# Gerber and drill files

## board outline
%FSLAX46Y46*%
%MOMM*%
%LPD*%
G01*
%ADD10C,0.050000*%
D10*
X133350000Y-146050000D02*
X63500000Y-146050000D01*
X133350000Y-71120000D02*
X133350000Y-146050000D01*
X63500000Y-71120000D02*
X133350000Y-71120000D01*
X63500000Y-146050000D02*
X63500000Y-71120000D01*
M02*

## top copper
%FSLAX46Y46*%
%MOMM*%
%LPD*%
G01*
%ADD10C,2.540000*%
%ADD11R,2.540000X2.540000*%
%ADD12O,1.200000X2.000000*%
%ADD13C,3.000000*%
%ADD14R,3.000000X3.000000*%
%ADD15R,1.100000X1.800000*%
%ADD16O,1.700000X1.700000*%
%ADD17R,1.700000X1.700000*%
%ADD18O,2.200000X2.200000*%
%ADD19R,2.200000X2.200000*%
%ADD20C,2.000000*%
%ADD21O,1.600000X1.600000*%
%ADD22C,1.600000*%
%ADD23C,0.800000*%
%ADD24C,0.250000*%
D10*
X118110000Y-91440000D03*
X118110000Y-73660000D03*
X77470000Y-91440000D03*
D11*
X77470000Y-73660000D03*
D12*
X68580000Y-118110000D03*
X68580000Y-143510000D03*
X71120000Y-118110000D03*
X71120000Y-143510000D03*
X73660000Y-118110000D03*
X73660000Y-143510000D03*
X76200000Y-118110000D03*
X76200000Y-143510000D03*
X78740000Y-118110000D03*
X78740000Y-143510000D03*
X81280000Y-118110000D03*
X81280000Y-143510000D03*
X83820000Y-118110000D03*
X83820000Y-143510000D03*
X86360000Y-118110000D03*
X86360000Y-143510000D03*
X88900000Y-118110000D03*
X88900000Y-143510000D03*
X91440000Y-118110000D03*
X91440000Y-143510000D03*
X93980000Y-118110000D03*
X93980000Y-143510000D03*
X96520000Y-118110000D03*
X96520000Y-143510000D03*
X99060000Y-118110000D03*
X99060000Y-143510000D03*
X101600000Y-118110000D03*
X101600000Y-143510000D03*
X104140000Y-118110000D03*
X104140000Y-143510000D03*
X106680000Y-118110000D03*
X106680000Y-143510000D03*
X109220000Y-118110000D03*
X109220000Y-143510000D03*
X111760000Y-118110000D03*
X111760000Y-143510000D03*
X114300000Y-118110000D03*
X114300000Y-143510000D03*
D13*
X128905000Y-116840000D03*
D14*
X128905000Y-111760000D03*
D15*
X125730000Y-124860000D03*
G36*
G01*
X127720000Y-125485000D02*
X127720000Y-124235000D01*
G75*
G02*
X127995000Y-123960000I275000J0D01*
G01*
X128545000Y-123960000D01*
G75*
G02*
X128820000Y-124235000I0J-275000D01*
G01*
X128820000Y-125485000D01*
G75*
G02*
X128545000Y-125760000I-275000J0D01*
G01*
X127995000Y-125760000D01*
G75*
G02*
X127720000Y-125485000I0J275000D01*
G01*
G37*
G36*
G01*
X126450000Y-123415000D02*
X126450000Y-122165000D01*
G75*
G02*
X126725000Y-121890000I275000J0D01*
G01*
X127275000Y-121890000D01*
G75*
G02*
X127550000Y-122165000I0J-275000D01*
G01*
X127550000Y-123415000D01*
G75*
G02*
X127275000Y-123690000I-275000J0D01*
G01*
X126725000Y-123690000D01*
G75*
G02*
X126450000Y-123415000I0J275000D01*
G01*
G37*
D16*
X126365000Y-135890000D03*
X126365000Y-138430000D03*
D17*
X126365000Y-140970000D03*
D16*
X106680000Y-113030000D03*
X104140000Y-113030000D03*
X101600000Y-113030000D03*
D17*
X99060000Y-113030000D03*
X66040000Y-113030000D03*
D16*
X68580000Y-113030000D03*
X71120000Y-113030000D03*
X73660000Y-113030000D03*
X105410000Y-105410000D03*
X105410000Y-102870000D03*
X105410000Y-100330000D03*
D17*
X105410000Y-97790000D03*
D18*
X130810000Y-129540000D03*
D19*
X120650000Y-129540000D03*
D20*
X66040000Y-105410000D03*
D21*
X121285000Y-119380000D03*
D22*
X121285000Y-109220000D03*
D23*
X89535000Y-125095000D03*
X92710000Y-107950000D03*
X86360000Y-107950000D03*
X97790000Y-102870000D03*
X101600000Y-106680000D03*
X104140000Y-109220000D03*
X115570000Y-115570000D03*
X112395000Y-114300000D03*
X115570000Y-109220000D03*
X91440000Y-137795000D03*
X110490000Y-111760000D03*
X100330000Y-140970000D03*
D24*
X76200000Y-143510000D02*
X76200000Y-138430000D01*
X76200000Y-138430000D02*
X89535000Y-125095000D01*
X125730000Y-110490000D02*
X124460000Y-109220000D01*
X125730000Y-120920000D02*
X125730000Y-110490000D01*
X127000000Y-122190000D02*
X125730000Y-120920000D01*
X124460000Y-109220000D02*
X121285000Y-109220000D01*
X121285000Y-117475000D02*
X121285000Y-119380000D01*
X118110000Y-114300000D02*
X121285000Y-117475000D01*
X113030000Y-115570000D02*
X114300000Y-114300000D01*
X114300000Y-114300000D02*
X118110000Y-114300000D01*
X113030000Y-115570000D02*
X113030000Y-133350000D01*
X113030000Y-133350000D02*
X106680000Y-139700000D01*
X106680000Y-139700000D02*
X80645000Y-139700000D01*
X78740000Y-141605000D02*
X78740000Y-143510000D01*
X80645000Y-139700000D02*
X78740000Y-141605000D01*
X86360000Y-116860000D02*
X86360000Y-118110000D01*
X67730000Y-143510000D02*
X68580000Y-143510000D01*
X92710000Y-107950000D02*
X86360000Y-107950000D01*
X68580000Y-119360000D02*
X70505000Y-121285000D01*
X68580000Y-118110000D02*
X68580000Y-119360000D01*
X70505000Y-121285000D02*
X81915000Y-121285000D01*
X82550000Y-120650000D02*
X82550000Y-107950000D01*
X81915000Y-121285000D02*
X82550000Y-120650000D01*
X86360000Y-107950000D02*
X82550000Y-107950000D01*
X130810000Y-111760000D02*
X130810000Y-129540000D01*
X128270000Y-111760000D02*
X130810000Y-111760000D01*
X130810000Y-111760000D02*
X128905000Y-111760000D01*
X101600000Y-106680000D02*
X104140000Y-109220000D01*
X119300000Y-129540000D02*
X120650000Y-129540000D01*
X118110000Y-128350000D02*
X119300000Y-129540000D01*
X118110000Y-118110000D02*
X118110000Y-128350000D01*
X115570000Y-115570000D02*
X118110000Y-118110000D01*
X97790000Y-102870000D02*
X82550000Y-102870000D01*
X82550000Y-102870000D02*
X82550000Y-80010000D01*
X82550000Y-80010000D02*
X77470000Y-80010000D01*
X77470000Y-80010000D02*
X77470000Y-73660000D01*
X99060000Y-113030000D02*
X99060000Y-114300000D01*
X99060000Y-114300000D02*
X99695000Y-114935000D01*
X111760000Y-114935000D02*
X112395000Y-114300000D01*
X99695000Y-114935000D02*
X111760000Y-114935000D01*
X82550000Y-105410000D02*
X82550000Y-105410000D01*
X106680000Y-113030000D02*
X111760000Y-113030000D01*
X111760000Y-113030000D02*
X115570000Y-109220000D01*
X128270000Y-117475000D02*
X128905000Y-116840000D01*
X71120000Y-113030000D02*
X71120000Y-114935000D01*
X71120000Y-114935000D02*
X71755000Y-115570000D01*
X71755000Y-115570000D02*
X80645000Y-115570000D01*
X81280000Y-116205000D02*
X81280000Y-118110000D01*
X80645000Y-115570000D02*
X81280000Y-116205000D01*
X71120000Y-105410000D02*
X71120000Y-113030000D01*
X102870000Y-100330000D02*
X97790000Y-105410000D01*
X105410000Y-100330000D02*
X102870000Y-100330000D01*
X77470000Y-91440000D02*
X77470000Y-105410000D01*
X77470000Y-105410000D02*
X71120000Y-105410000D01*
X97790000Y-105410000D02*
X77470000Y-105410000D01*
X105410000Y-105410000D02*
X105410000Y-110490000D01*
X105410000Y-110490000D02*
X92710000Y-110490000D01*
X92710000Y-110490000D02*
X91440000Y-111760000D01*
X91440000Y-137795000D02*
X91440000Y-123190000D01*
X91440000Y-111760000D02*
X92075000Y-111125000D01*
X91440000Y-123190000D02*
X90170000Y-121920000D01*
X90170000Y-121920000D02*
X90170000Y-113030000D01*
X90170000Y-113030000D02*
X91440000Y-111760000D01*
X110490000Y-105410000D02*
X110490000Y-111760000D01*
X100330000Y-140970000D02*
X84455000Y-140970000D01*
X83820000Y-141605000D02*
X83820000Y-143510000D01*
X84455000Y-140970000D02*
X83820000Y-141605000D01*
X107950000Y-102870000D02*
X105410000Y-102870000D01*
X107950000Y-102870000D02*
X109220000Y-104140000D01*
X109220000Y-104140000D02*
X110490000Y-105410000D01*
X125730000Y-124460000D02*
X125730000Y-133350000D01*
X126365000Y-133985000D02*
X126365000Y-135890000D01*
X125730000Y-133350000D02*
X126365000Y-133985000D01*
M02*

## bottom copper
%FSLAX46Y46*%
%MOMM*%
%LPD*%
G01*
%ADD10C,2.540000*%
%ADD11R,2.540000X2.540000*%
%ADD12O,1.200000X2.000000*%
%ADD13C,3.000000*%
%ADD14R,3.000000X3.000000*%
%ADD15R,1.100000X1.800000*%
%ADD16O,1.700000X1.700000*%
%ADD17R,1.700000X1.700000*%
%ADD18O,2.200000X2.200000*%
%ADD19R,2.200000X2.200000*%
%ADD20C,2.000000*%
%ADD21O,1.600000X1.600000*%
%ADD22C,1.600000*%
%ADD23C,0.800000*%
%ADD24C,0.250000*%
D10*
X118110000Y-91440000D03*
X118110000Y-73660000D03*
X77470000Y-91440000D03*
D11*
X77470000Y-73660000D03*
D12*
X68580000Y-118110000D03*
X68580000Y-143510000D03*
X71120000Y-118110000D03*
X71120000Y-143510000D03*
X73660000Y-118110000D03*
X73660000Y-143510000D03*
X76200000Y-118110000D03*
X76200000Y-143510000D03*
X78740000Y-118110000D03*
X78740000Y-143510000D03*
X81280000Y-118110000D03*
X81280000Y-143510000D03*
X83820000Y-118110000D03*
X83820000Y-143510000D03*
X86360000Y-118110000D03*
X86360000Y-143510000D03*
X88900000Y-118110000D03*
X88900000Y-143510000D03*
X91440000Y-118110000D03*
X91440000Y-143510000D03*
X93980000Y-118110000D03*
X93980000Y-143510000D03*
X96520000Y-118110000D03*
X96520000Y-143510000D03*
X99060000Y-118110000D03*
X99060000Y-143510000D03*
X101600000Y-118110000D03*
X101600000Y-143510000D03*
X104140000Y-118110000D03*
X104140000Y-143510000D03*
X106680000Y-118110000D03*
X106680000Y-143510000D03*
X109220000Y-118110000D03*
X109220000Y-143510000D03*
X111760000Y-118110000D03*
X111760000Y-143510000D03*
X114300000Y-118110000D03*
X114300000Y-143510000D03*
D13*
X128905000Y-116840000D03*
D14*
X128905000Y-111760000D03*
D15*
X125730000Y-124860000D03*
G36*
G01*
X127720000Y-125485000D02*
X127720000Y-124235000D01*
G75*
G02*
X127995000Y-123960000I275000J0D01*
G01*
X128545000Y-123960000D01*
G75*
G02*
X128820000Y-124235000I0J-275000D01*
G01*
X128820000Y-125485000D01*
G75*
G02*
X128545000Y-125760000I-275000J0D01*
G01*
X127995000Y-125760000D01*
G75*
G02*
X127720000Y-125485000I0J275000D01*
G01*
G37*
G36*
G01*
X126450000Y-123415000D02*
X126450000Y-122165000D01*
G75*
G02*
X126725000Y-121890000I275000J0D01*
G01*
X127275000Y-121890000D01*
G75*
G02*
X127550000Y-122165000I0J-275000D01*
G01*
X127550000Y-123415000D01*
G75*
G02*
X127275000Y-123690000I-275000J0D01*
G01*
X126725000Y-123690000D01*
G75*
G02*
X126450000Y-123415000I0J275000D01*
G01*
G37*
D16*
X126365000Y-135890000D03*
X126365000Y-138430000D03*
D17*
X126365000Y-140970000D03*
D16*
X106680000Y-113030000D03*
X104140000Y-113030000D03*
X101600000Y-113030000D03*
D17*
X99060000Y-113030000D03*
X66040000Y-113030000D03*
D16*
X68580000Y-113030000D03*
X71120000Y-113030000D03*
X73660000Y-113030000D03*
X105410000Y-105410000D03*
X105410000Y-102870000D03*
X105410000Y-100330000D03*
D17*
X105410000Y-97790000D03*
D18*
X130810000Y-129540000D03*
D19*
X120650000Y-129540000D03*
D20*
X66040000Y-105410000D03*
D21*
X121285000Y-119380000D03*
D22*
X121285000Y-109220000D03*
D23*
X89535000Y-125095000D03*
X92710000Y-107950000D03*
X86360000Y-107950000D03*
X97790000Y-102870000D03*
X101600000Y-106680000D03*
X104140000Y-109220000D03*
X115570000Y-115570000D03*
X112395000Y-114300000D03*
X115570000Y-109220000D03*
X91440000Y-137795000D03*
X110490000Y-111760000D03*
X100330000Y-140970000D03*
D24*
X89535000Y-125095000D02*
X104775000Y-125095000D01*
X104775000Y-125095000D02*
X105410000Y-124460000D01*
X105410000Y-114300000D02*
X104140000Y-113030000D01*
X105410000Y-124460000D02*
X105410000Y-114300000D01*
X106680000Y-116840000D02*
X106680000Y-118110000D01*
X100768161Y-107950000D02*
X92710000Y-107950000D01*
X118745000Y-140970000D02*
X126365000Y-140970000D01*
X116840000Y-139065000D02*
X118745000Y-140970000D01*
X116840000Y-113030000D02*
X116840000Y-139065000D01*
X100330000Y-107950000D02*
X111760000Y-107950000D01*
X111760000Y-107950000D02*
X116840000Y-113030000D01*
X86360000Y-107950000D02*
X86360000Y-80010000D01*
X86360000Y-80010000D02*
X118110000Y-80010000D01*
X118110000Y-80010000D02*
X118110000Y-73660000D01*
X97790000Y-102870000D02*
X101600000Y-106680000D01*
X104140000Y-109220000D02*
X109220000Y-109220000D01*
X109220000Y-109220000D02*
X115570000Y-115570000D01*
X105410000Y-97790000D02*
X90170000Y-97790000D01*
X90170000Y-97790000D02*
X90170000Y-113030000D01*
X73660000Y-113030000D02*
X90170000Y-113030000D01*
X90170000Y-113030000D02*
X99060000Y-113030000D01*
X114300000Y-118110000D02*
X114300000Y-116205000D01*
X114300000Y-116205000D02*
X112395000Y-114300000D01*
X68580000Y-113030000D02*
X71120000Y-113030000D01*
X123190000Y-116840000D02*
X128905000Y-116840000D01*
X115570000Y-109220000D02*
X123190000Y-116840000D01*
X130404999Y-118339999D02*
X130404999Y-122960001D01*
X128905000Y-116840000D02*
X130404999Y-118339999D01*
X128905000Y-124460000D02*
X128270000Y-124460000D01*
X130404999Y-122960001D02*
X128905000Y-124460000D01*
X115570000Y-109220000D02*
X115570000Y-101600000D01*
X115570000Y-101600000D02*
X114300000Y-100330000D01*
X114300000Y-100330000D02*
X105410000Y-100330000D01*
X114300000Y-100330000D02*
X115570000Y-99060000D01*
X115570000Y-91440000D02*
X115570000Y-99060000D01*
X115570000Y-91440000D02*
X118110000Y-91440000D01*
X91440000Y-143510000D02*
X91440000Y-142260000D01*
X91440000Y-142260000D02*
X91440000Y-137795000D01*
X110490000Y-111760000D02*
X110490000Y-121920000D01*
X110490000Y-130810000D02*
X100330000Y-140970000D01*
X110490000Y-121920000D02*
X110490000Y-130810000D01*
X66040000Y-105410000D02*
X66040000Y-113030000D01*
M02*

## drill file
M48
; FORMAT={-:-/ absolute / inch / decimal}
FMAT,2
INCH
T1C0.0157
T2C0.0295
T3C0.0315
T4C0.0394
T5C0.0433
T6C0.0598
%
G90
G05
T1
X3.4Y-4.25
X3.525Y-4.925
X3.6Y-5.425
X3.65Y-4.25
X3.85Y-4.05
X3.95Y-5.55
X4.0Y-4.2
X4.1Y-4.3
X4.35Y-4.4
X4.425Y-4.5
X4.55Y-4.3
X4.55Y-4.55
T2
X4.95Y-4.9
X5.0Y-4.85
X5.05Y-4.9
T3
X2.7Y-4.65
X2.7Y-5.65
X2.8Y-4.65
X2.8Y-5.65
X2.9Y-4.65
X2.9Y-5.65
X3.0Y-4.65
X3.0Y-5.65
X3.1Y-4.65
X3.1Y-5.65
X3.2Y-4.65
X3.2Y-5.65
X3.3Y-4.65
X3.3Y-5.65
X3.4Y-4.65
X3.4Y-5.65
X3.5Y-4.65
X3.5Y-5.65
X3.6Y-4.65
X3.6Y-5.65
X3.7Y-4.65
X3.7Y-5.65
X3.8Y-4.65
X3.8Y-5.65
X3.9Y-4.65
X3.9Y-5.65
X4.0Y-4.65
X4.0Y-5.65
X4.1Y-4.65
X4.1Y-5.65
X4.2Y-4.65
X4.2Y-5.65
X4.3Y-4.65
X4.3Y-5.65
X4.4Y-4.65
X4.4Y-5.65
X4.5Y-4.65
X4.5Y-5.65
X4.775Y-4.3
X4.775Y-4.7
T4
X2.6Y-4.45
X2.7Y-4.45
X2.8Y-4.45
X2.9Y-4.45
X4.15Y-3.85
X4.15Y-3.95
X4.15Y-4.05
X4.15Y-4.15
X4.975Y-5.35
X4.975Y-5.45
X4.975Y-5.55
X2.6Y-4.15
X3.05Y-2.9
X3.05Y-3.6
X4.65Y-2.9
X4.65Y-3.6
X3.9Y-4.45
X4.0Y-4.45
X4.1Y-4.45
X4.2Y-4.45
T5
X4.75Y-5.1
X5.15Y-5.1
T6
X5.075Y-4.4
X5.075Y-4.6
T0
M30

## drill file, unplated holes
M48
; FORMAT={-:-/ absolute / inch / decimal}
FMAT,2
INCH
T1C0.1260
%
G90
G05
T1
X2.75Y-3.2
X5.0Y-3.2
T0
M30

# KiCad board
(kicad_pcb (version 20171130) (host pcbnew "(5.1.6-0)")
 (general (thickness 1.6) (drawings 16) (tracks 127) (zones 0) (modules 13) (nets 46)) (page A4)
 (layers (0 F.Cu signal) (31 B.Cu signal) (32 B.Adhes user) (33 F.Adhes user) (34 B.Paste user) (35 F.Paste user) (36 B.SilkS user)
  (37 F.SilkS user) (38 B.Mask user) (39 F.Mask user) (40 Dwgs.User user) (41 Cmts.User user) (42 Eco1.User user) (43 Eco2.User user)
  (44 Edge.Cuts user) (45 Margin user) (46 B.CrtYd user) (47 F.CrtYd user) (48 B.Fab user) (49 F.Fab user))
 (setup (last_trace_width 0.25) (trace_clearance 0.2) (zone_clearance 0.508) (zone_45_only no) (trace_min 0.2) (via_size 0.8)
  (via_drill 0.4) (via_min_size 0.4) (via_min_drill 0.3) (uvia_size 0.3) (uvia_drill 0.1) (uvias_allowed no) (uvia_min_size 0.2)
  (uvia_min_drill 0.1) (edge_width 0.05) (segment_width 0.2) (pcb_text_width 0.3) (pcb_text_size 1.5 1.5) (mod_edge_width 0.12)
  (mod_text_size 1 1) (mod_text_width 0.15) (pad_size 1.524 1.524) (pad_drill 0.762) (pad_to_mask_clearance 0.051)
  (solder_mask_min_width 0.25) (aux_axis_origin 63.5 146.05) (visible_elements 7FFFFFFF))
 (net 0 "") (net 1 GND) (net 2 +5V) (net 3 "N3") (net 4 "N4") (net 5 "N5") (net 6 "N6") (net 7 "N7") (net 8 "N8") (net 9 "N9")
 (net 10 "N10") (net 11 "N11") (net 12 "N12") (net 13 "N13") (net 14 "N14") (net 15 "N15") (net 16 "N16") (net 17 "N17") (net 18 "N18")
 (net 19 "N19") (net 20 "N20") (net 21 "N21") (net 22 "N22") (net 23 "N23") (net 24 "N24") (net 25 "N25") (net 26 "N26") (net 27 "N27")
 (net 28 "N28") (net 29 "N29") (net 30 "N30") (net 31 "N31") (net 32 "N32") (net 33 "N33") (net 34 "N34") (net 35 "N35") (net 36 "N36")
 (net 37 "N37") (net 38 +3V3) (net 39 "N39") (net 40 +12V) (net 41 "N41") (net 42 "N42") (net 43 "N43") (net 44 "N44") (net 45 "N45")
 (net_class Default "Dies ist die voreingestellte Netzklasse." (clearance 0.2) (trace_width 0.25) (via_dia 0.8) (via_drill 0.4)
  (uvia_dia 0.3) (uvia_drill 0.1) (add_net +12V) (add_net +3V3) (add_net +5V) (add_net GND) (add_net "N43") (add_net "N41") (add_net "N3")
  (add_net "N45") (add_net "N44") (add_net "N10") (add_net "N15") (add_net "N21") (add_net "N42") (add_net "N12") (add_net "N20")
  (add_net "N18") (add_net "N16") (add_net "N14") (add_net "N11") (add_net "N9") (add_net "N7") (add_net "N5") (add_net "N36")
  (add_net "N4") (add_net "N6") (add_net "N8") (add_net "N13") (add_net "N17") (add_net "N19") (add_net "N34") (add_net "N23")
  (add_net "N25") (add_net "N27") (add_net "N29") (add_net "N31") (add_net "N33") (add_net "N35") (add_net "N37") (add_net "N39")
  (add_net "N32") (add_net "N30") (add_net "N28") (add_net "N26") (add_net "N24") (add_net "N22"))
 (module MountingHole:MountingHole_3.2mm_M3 (layer F.Cu) (at 69.85 81.28)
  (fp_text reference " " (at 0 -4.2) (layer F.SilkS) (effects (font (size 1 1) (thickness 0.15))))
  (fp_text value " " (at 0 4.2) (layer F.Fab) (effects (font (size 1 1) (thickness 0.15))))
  (pad 1 np_thru_hole circle (at 0 0) (size 3.2 3.2) (drill 3.2) (layers *.Cu *.Mask)))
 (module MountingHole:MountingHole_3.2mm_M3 (layer F.Cu) (at 127 81.28)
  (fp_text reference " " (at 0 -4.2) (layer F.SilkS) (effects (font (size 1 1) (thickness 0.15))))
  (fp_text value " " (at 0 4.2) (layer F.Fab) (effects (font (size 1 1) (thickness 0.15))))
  (pad 1 np_thru_hole circle (at 0 0) (size 3.2 3.2) (drill 3.2) (layers *.Cu *.Mask)))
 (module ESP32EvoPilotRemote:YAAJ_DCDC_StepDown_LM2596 (layer F.Cu) (at 77.47 73.66)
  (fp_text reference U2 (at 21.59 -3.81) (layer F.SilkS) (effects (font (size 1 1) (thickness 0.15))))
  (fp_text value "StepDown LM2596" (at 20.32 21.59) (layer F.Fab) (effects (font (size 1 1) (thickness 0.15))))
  (pad 3 thru_hole circle (at 40.64 17.78) (size 2.54 2.54) (drill 1) (layers *.Cu *.Mask) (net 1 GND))
  (pad 4 thru_hole circle (at 40.64 0) (size 2.54 2.54) (drill 1) (layers *.Cu *.Mask) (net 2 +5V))
  (pad 2 thru_hole circle (at 0 17.78) (size 2.54 2.54) (drill 1) (layers *.Cu *.Mask) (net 1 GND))
  (pad 1 thru_hole rect (at 0 0) (size 2.54 2.54) (drill 1) (layers *.Cu *.Mask) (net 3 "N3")))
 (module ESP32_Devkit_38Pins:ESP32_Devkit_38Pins (layer F.Cu) (at 91.44 130.81 180)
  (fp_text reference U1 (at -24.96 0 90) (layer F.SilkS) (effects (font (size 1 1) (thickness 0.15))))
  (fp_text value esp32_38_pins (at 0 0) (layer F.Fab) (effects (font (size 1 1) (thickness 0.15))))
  (pad 19 thru_hole oval (at 22.86 12.7 180) (size 1.2 2) (drill 0.8) (layers *.Cu *.Mask) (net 2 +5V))
  (pad 20 thru_hole oval (at 22.86 -12.7 180) (size 1.2 2) (drill 0.8) (layers *.Cu *.Mask) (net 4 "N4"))
  (pad 18 thru_hole oval (at 20.32 12.7 180) (size 1.2 2) (drill 0.8) (layers *.Cu *.Mask) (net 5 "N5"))
  (pad 21 thru_hole oval (at 20.32 -12.7 180) (size 1.2 2) (drill 0.8) (layers *.Cu *.Mask) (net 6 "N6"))
  (pad 17 thru_hole oval (at 17.78 12.7 180) (size 1.2 2) (drill 0.8) (layers *.Cu *.Mask) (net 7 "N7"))
  (pad 22 thru_hole oval (at 17.78 -12.7 180) (size 1.2 2) (drill 0.8) (layers *.Cu *.Mask) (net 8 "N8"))
  (pad 16 thru_hole oval (at 15.24 12.7 180) (size 1.2 2) (drill 0.8) (layers *.Cu *.Mask) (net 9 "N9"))
  (pad 23 thru_hole oval (at 15.24 -12.7 180) (size 1.2 2) (drill 0.8) (layers *.Cu *.Mask) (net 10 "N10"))
  (pad 15 thru_hole oval (at 12.7 12.7 180) (size 1.2 2) (drill 0.8) (layers *.Cu *.Mask) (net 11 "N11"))
  (pad 24 thru_hole oval (at 12.7 -12.7 180) (size 1.2 2) (drill 0.8) (layers *.Cu *.Mask) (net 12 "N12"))
  (pad 14 thru_hole oval (at 10.16 12.7 180) (size 1.2 2) (drill 0.8) (layers *.Cu *.Mask) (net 1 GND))
  (pad 25 thru_hole oval (at 10.16 -12.7 180) (size 1.2 2) (drill 0.8) (layers *.Cu *.Mask) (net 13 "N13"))
  (pad 13 thru_hole oval (at 7.62 12.7 180) (size 1.2 2) (drill 0.8) (layers *.Cu *.Mask) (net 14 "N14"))
  (pad 26 thru_hole oval (at 7.62 -12.7 180) (size 1.2 2) (drill 0.8) (layers *.Cu *.Mask) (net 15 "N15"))
  (pad 12 thru_hole oval (at 5.08 12.7 180) (size 1.2 2) (drill 0.8) (layers *.Cu *.Mask) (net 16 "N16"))
  (pad 27 thru_hole oval (at 5.08 -12.7 180) (size 1.2 2) (drill 0.8) (layers *.Cu *.Mask) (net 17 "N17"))
  (pad 11 thru_hole oval (at 2.54 12.7 180) (size 1.2 2) (drill 0.8) (layers *.Cu *.Mask) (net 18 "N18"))
  (pad 28 thru_hole oval (at 2.54 -12.7 180) (size 1.2 2) (drill 0.8) (layers *.Cu *.Mask) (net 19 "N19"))
  (pad 10 thru_hole oval (at 0 12.7 180) (size 1.2 2) (drill 0.8) (layers *.Cu *.Mask) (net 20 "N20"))
  (pad 29 thru_hole oval (at 0 -12.7 180) (size 1.2 2) (drill 0.8) (layers *.Cu *.Mask) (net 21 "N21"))
  (pad 9 thru_hole oval (at -2.54 12.7 180) (size 1.2 2) (drill 0.8) (layers *.Cu *.Mask) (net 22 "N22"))
  (pad 30 thru_hole oval (at -2.54 -12.7 180) (size 1.2 2) (drill 0.8) (layers *.Cu *.Mask) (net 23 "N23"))
  (pad 8 thru_hole oval (at -5.08 12.7 180) (size 1.2 2) (drill 0.8) (layers *.Cu *.Mask) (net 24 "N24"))
  (pad 31 thru_hole oval (at -5.08 -12.7 180) (size 1.2 2) (drill 0.8) (layers *.Cu *.Mask) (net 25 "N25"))
  (pad 7 thru_hole oval (at -7.62 12.7 180) (size 1.2 2) (drill 0.8) (layers *.Cu *.Mask) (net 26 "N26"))
  (pad 32 thru_hole oval (at -7.62 -12.7 180) (size 1.2 2) (drill 0.8) (layers *.Cu *.Mask) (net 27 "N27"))
  (pad 6 thru_hole oval (at -10.16 12.7 180) (size 1.2 2) (drill 0.8) (layers *.Cu *.Mask) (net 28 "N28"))
  (pad 33 thru_hole oval (at -10.16 -12.7 180) (size 1.2 2) (drill 0.8) (layers *.Cu *.Mask) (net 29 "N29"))
  (pad 5 thru_hole oval (at -12.7 12.7 180) (size 1.2 2) (drill 0.8) (layers *.Cu *.Mask) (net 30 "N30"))
  (pad 34 thru_hole oval (at -12.7 -12.7 180) (size 1.2 2) (drill 0.8) (layers *.Cu *.Mask) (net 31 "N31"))
  (pad 4 thru_hole oval (at -15.24 12.7 180) (size 1.2 2) (drill 0.8) (layers *.Cu *.Mask) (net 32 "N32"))
  (pad 35 thru_hole oval (at -15.24 -12.7 180) (size 1.2 2) (drill 0.8) (layers *.Cu *.Mask) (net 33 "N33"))
  (pad 3 thru_hole oval (at -17.78 12.7 180) (size 1.2 2) (drill 0.8) (layers *.Cu *.Mask) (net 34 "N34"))
  (pad 36 thru_hole oval (at -17.78 -12.7 180) (size 1.2 2) (drill 0.8) (layers *.Cu *.Mask) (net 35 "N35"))
  (pad 2 thru_hole oval (at -20.32 12.7 180) (size 1.2 2) (drill 0.8) (layers *.Cu *.Mask) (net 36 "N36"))
  (pad 37 thru_hole oval (at -20.32 -12.7 180) (size 1.2 2) (drill 0.8) (layers *.Cu *.Mask) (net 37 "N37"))
  (pad 1 thru_hole oval (at -22.86 12.7 180) (size 1.2 2) (drill 0.8) (layers *.Cu *.Mask) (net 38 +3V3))
  (pad 38 thru_hole oval (at -22.86 -12.7 180) (size 1.2 2) (drill 0.8) (layers *.Cu *.Mask) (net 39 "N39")))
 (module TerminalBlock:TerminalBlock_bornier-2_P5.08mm (layer F.Cu) (at 128.905 111.76 270)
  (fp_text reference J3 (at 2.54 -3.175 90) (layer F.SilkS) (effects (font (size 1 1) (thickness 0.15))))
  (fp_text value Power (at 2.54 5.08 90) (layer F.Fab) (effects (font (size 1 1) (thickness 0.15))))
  (pad 2 thru_hole circle (at 5.08 0 270) (size 3 3) (drill 1.52) (layers *.Cu *.Mask) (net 1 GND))
  (pad 1 thru_hole rect (at 0 0 270) (size 3 3) (drill 1.52) (layers *.Cu *.Mask) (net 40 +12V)))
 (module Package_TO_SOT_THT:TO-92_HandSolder (layer F.Cu) (at 125.73 124.46)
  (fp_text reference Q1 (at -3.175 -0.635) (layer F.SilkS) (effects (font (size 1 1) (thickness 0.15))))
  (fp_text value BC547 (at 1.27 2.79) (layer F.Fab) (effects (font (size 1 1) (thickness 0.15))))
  (pad 1 thru_hole rect (at 0 0) (size 1.1 1.8) (drill 0.75 (offset 0 0.4)) (layers *.Cu *.Mask) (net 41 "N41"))
  (pad 3 thru_hole roundrect (at 2.54 0) (size 1.1 1.8) (drill 0.75 (offset 0 0.4)) (layers *.Cu *.Mask) (roundrect_rratio 0.25) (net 1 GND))
  (pad 2 thru_hole roundrect (at 1.27 -1.27) (size 1.1 1.8) (drill 0.75 (offset 0 -0.4)) (layers *.Cu *.Mask) (roundrect_rratio 0.25)
   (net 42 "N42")))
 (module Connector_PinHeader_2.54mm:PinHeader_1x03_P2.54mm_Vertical (layer F.Cu) (at 126.365 140.97 180)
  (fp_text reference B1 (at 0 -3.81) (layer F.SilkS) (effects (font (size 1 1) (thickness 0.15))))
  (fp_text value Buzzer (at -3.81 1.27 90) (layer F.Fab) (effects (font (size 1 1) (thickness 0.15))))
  (pad 3 thru_hole oval (at 0 5.08 180) (size 1.7 1.7) (drill 1) (layers *.Cu *.Mask) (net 41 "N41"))
  (pad 2 thru_hole oval (at 0 2.54 180) (size 1.7 1.7) (drill 1) (layers *.Cu *.Mask) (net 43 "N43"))
  (pad 1 thru_hole rect (at 0 0 180) (size 1.7 1.7) (drill 1) (layers *.Cu *.Mask) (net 2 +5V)))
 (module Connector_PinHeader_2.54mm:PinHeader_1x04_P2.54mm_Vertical (layer F.Cu) (at 99.06 113.03 90)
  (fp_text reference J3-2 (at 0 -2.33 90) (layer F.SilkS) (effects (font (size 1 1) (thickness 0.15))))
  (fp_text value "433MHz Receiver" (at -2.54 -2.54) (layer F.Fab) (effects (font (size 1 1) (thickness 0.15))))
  (pad 4 thru_hole oval (at 0 7.62 90) (size 1.7 1.7) (drill 1) (layers *.Cu *.Mask) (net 1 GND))
  (pad 3 thru_hole oval (at 0 5.08 90) (size 1.7 1.7) (drill 1) (layers *.Cu *.Mask) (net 10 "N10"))
  (pad 2 thru_hole oval (at 0 2.54 90) (size 1.7 1.7) (drill 1) (layers *.Cu *.Mask) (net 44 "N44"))
  (pad 1 thru_hole rect (at 0 0 90) (size 1.7 1.7) (drill 1) (layers *.Cu *.Mask) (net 38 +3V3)))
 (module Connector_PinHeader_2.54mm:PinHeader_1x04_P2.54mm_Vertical (layer F.Cu) (at 66.04 113.03 90)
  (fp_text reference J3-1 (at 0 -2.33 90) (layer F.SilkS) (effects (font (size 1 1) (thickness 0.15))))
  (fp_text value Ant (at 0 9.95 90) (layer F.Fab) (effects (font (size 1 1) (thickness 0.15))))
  (pad 1 thru_hole rect (at 0 0 90) (size 1.7 1.7) (drill 1) (layers *.Cu *.Mask) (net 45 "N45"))
  (pad 2 thru_hole oval (at 0 2.54 90) (size 1.7 1.7) (drill 1) (layers *.Cu *.Mask) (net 1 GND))
  (pad 3 thru_hole oval (at 0 5.08 90) (size 1.7 1.7) (drill 1) (layers *.Cu *.Mask) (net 1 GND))
  (pad 4 thru_hole oval (at 0 7.62 90) (size 1.7 1.7) (drill 1) (layers *.Cu *.Mask) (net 38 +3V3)))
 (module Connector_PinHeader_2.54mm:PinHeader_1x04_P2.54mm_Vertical (layer F.Cu) (at 105.41 97.79)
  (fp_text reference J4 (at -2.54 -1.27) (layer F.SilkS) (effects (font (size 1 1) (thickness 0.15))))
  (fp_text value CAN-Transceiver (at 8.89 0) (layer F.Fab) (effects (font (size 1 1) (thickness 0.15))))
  (pad 4 thru_hole oval (at 0 7.62) (size 1.7 1.7) (drill 1) (layers *.Cu *.Mask) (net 21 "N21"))
  (pad 3 thru_hole oval (at 0 5.08) (size 1.7 1.7) (drill 1) (layers *.Cu *.Mask) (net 15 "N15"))
  (pad 2 thru_hole oval (at 0 2.54) (size 1.7 1.7) (drill 1) (layers *.Cu *.Mask) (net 1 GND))
  (pad 1 thru_hole rect (at 0 0) (size 1.7 1.7) (drill 1) (layers *.Cu *.Mask) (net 38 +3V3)))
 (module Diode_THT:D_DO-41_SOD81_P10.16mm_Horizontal (layer F.Cu) (at 120.65 129.54)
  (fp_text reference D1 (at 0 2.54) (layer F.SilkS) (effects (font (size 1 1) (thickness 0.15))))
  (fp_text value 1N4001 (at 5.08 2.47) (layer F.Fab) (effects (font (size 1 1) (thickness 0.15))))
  (pad 2 thru_hole oval (at 10.16 0) (size 2.2 2.2) (drill 1.1) (layers *.Cu *.Mask) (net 40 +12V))
  (pad 1 thru_hole rect (at 0 0) (size 2.2 2.2) (drill 1.1) (layers *.Cu *.Mask) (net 3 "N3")))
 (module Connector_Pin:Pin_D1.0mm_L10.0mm (layer F.Cu) (at 66.04 105.41)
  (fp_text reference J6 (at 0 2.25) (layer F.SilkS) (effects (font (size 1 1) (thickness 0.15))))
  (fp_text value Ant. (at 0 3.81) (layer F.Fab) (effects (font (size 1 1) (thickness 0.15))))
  (pad 1 thru_hole circle (at 0 0) (size 2 2) (drill 1) (layers *.Cu *.Mask) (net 45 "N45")))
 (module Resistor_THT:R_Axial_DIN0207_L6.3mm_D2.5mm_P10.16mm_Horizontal (layer F.Cu) (at 121.285 109.22 270)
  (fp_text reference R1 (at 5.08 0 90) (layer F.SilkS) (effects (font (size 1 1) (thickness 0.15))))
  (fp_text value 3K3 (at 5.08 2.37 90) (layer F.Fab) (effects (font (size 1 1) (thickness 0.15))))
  (pad 2 thru_hole oval (at 10.16 0 270) (size 1.6 1.6) (drill 0.8) (layers *.Cu *.Mask) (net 12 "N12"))
  (pad 1 thru_hole circle (at 0 0 270) (size 1.6 1.6) (drill 0.8) (layers *.Cu *.Mask) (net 42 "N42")))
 (gr_line (start 133.35 146.05) (end 63.5 146.05) (layer Edge.Cuts) (width 0.05))
 (gr_line (start 133.35 71.12) (end 133.35 146.05) (layer Edge.Cuts) (width 0.05))
 (gr_line (start 63.5 71.12) (end 133.35 71.12) (layer Edge.Cuts) (width 0.05))
 (gr_line (start 63.5 146.05) (end 63.5 71.12) (layer Edge.Cuts) (width 0.05))
 (segment (start 76.2 143.51) (end 76.2 138.43) (width 0.25) (layer F.Cu) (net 10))
 (via (at 89.535 125.095) (size 0.8) (drill 0.4) (layers F.Cu B.Cu) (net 10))
 (segment (start 76.2 138.43) (end 89.535 125.095) (width 0.25) (layer F.Cu) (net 10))
 (segment (start 89.535 125.095) (end 104.775 125.095) (width 0.25) (layer B.Cu) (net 10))
 (segment (start 104.775 125.095) (end 105.41 124.46) (width 0.25) (layer B.Cu) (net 10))
 (segment (start 105.41 114.3) (end 104.14 113.03) (width 0.25) (layer B.Cu) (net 10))
 (segment (start 105.41 124.46) (end 105.41 114.3) (width 0.25) (layer B.Cu) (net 10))
 (segment (start 125.73 110.49) (end 124.46 109.22) (width 0.25) (layer F.Cu) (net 42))
 (segment (start 125.73 120.92) (end 125.73 110.49) (width 0.25) (layer F.Cu) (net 42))
 (segment (start 127 122.19) (end 125.73 120.92) (width 0.25) (layer F.Cu) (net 42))
 (segment (start 124.46 109.22) (end 121.285 109.22) (width 0.25) (layer F.Cu) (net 42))
 (segment (start 121.285 117.475) (end 121.285 119.38) (width 0.25) (layer F.Cu) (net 12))
 (segment (start 118.11 114.3) (end 121.285 117.475) (width 0.25) (layer F.Cu) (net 12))
 (segment (start 113.03 115.57) (end 114.3 114.3) (width 0.25) (layer F.Cu) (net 12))
 (segment (start 114.3 114.3) (end 118.11 114.3) (width 0.25) (layer F.Cu) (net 12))
 (segment (start 113.03 115.57) (end 113.03 133.35) (width 0.25) (layer F.Cu) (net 12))
 (segment (start 113.03 133.35) (end 106.68 139.7) (width 0.25) (layer F.Cu) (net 12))
 (segment (start 106.68 139.7) (end 80.645 139.7) (width 0.25) (layer F.Cu) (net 12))
 (segment (start 78.74 141.605) (end 78.74 143.51) (width 0.25) (layer F.Cu) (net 12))
 (segment (start 80.645 139.7) (end 78.74 141.605) (width 0.25) (layer F.Cu) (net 12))
 (segment (start 106.68 116.84) (end 106.68 118.11) (width 0.25) (layer B.Cu) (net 32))
 (segment (start 86.36 116.86) (end 86.36 118.11) (width 0.25) (layer F.Cu) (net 16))
 (segment (start 67.73 143.51) (end 68.58 143.51) (width 0.25) (layer F.Cu) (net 4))
 (segment (start 100.768161 107.95) (end 92.71 107.95) (width 0.25) (layer B.Cu) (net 2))
 (via (at 92.71 107.95) (size 0.8) (drill 0.4) (layers F.Cu B.Cu) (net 2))
 (segment (start 92.71 107.95) (end 86.36 107.95) (width 0.25) (layer F.Cu) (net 2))
 (segment (start 68.58 119.36) (end 70.505 121.285) (width 0.25) (layer F.Cu) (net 2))
 (segment (start 68.58 118.11) (end 68.58 119.36) (width 0.25) (layer F.Cu) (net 2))
 (segment (start 70.505 121.285) (end 81.915 121.285) (width 0.25) (layer F.Cu) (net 2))
 (segment (start 82.55 120.65) (end 82.55 107.95) (width 0.25) (layer F.Cu) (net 2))
 (segment (start 81.915 121.285) (end 82.55 120.65) (width 0.25) (layer F.Cu) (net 2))
 (segment (start 118.745 140.97) (end 126.365 140.97) (width 0.25) (layer B.Cu) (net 2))
 (segment (start 116.84 139.065) (end 118.745 140.97) (width 0.25) (layer B.Cu) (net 2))
 (segment (start 116.84 113.03) (end 116.84 139.065) (width 0.25) (layer B.Cu) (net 2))
 (segment (start 100.33 107.95) (end 111.76 107.95) (width 0.25) (layer B.Cu) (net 2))
 (segment (start 111.76 107.95) (end 116.84 113.03) (width 0.25) (layer B.Cu) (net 2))
 (segment (start 86.36 107.95) (end 82.55 107.95) (width 0.25) (layer F.Cu) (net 2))
 (via (at 86.36 107.95) (size 0.8) (drill 0.4) (layers F.Cu B.Cu) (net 2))
 (segment (start 86.36 107.95) (end 86.36 80.01) (width 0.25) (layer B.Cu) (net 2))
 (segment (start 86.36 80.01) (end 118.11 80.01) (width 0.25) (layer B.Cu) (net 2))
 (segment (start 118.11 80.01) (end 118.11 73.66) (width 0.25) (layer B.Cu) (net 2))
 (segment (start 130.81 111.76) (end 130.81 129.54) (width 0.25) (layer F.Cu) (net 40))
 (segment (start 128.27 111.76) (end 130.81 111.76) (width 0.25) (layer F.Cu) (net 40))
 (segment (start 130.81 111.76) (end 128.905 111.76) (width 0.25) (layer F.Cu) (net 40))
 (via (at 97.79 102.87) (size 0.8) (drill 0.4) (layers F.Cu B.Cu) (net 3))
 (segment (start 97.79 102.87) (end 101.6 106.68) (width 0.25) (layer B.Cu) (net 3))
 (via (at 101.6 106.68) (size 0.8) (drill 0.4) (layers F.Cu B.Cu) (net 3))
 (segment (start 101.6 106.68) (end 104.14 109.22) (width 0.25) (layer F.Cu) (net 3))
 (via (at 104.14 109.22) (size 0.8) (drill 0.4) (layers F.Cu B.Cu) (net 3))
 (segment (start 104.14 109.22) (end 109.22 109.22) (width 0.25) (layer B.Cu) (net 3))
 (segment (start 109.22 109.22) (end 115.57 115.57) (width 0.25) (layer B.Cu) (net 3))
 (via (at 115.57 115.57) (size 0.8) (drill 0.4) (layers F.Cu B.Cu) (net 3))
 (segment (start 119.3 129.54) (end 120.65 129.54) (width 0.25) (layer F.Cu) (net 3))
 (segment (start 118.11 128.35) (end 119.3 129.54) (width 0.25) (layer F.Cu) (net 3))
 (segment (start 118.11 118.11) (end 118.11 128.35) (width 0.25) (layer F.Cu) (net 3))
 (segment (start 115.57 115.57) (end 118.11 118.11) (width 0.25) (layer F.Cu) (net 3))
 (segment (start 97.79 102.87) (end 82.55 102.87) (width 0.25) (layer F.Cu) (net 3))
 (segment (start 82.55 102.87) (end 82.55 80.01) (width 0.25) (layer F.Cu) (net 3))
 (segment (start 82.55 80.01) (end 77.47 80.01) (width 0.25) (layer F.Cu) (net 3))
 (segment (start 77.47 80.01) (end 77.47 73.66) (width 0.25) (layer F.Cu) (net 3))
 (segment (start 105.41 97.79) (end 90.17 97.79) (width 0.25) (layer B.Cu) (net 38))
 (segment (start 90.17 97.79) (end 90.17 113.03) (width 0.25) (layer B.Cu) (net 38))
 (segment (start 73.66 113.03) (end 90.17 113.03) (width 0.25) (layer B.Cu) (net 38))
 (segment (start 90.17 113.03) (end 99.06 113.03) (width 0.25) (layer B.Cu) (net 38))
 (segment (start 114.3 118.11) (end 114.3 116.205) (width 0.25) (layer B.Cu) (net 38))
 (segment (start 114.3 116.205) (end 112.395 114.3) (width 0.25) (layer B.Cu) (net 38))
 (via (at 112.395 114.3) (size 0.8) (drill 0.4) (layers F.Cu B.Cu) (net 38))
 (segment (start 99.06 113.03) (end 99.06 114.3) (width 0.25) (layer F.Cu) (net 38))
 (segment (start 99.06 114.3) (end 99.695 114.935) (width 0.25) (layer F.Cu) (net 38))
 (segment (start 111.76 114.935) (end 112.395 114.3) (width 0.25) (layer F.Cu) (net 38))
 (segment (start 99.695 114.935) (end 111.76 114.935) (width 0.25) (layer F.Cu) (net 38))
 (segment (start 68.58 113.03) (end 71.12 113.03) (width 0.25) (layer B.Cu) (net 1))
 (segment (start 82.55 105.41) (end 82.55 105.41) (width 0.25) (layer F.Cu) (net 1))
 (segment (start 106.68 113.03) (end 111.76 113.03) (width 0.25) (layer F.Cu) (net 1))
 (segment (start 111.76 113.03) (end 115.57 109.22) (width 0.25) (layer F.Cu) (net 1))
 (via (at 115.57 109.22) (size 0.8) (drill 0.4) (layers F.Cu B.Cu) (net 1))
 (segment (start 123.19 116.84) (end 128.905 116.84) (width 0.25) (layer B.Cu) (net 1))
 (segment (start 115.57 109.22) (end 123.19 116.84) (width 0.25) (layer B.Cu) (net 1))
 (segment (start 128.27 117.475) (end 128.905 116.84) (width 0.25) (layer F.Cu) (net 1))
 (segment (start 130.404999 118.339999) (end 130.404999 122.960001) (width 0.25) (layer B.Cu) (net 1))
 (segment (start 128.905 116.84) (end 130.404999 118.339999) (width 0.25) (layer B.Cu) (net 1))
 (segment (start 128.905 124.46) (end 128.27 124.46) (width 0.25) (layer B.Cu) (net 1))
 (segment (start 130.404999 122.960001) (end 128.905 124.46) (width 0.25) (layer B.Cu) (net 1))
 (segment (start 71.12 113.03) (end 71.12 114.935) (width 0.25) (layer F.Cu) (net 1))
 (segment (start 71.12 114.935) (end 71.755 115.57) (width 0.25) (layer F.Cu) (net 1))
 (segment (start 71.755 115.57) (end 80.645 115.57) (width 0.25) (layer F.Cu) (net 1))
 (segment (start 81.28 116.205) (end 81.28 118.11) (width 0.25) (layer F.Cu) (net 1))
 (segment (start 80.645 115.57) (end 81.28 116.205) (width 0.25) (layer F.Cu) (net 1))
 (segment (start 115.57 109.22) (end 115.57 101.6) (width 0.25) (layer B.Cu) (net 1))
 (segment (start 115.57 101.6) (end 114.3 100.33) (width 0.25) (layer B.Cu) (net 1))
 (segment (start 114.3 100.33) (end 105.41 100.33) (width 0.25) (layer B.Cu) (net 1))
 (segment (start 114.3 100.33) (end 115.57 99.06) (width 0.25) (layer B.Cu) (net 1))
 (segment (start 115.57 91.44) (end 115.57 99.06) (width 0.25) (layer B.Cu) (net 1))
 (segment (start 115.57 91.44) (end 118.11 91.44) (width 0.25) (layer B.Cu) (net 1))
 (segment (start 71.12 105.41) (end 71.12 113.03) (width 0.25) (layer F.Cu) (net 1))
 (segment (start 102.87 100.33) (end 97.79 105.41) (width 0.25) (layer F.Cu) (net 1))
 (segment (start 105.41 100.33) (end 102.87 100.33) (width 0.25) (layer F.Cu) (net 1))
 (segment (start 77.47 91.44) (end 77.47 105.41) (width 0.25) (layer F.Cu) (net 1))
 (segment (start 77.47 105.41) (end 71.12 105.41) (width 0.25) (layer F.Cu) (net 1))
 (segment (start 97.79 105.41) (end 77.47 105.41) (width 0.25) (layer F.Cu) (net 1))
 (segment (start 105.41 105.41) (end 105.41 110.49) (width 0.25) (layer F.Cu) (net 21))
 (segment (start 105.41 110.49) (end 92.71 110.49) (width 0.25) (layer F.Cu) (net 21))
 (segment (start 92.71 110.49) (end 91.44 111.76) (width 0.25) (layer F.Cu) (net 21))
 (segment (start 91.44 143.51) (end 91.44 142.26) (width 0.25) (layer B.Cu) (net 21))
 (via (at 91.44 137.795) (size 0.8) (drill 0.4) (layers F.Cu B.Cu) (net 21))
 (segment (start 91.44 142.26) (end 91.44 137.795) (width 0.25) (layer B.Cu) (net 21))
 (segment (start 91.44 137.795) (end 91.44 123.19) (width 0.25) (layer F.Cu) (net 21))
 (segment (start 91.44 111.76) (end 92.075 111.125) (width 0.25) (layer F.Cu) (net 21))
 (segment (start 91.44 123.19) (end 90.17 121.92) (width 0.25) (layer F.Cu) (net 21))
 (segment (start 90.17 121.92) (end 90.17 113.03) (width 0.25) (layer F.Cu) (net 21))
 (segment (start 90.17 113.03) (end 91.44 111.76) (width 0.25) (layer F.Cu) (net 21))
 (via (at 110.49 111.76) (size 0.8) (drill 0.4) (layers F.Cu B.Cu) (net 15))
 (segment (start 110.49 105.41) (end 110.49 111.76) (width 0.25) (layer F.Cu) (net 15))
 (segment (start 110.49 111.76) (end 110.49 121.92) (width 0.25) (layer B.Cu) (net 15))
 (segment (start 110.49 130.81) (end 100.33 140.97) (width 0.25) (layer B.Cu) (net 15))
 (segment (start 110.49 121.92) (end 110.49 130.81) (width 0.25) (layer B.Cu) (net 15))
 (via (at 100.33 140.97) (size 0.8) (drill 0.4) (layers F.Cu B.Cu) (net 15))
 (segment (start 100.33 140.97) (end 84.455 140.97) (width 0.25) (layer F.Cu) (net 15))
 (segment (start 83.82 141.605) (end 83.82 143.51) (width 0.25) (layer F.Cu) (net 15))
 (segment (start 84.455 140.97) (end 83.82 141.605) (width 0.25) (layer F.Cu) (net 15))
 (segment (start 107.95 102.87) (end 105.41 102.87) (width 0.25) (layer F.Cu) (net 15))
 (segment (start 107.95 102.87) (end 109.22 104.14) (width 0.25) (layer F.Cu) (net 15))
 (segment (start 109.22 104.14) (end 110.49 105.41) (width 0.25) (layer F.Cu) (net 15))
 (segment (start 66.04 105.41) (end 66.04 113.03) (width 0.25) (layer B.Cu) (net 45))
 (segment (start 125.73 124.46) (end 125.73 133.35) (width 0.25) (layer F.Cu) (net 41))
 (segment (start 126.365 133.985) (end 126.365 135.89) (width 0.25) (layer F.Cu) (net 41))
 (segment (start 125.73 133.35) (end 126.365 133.985) (width 0.25) (layer F.Cu) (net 41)))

